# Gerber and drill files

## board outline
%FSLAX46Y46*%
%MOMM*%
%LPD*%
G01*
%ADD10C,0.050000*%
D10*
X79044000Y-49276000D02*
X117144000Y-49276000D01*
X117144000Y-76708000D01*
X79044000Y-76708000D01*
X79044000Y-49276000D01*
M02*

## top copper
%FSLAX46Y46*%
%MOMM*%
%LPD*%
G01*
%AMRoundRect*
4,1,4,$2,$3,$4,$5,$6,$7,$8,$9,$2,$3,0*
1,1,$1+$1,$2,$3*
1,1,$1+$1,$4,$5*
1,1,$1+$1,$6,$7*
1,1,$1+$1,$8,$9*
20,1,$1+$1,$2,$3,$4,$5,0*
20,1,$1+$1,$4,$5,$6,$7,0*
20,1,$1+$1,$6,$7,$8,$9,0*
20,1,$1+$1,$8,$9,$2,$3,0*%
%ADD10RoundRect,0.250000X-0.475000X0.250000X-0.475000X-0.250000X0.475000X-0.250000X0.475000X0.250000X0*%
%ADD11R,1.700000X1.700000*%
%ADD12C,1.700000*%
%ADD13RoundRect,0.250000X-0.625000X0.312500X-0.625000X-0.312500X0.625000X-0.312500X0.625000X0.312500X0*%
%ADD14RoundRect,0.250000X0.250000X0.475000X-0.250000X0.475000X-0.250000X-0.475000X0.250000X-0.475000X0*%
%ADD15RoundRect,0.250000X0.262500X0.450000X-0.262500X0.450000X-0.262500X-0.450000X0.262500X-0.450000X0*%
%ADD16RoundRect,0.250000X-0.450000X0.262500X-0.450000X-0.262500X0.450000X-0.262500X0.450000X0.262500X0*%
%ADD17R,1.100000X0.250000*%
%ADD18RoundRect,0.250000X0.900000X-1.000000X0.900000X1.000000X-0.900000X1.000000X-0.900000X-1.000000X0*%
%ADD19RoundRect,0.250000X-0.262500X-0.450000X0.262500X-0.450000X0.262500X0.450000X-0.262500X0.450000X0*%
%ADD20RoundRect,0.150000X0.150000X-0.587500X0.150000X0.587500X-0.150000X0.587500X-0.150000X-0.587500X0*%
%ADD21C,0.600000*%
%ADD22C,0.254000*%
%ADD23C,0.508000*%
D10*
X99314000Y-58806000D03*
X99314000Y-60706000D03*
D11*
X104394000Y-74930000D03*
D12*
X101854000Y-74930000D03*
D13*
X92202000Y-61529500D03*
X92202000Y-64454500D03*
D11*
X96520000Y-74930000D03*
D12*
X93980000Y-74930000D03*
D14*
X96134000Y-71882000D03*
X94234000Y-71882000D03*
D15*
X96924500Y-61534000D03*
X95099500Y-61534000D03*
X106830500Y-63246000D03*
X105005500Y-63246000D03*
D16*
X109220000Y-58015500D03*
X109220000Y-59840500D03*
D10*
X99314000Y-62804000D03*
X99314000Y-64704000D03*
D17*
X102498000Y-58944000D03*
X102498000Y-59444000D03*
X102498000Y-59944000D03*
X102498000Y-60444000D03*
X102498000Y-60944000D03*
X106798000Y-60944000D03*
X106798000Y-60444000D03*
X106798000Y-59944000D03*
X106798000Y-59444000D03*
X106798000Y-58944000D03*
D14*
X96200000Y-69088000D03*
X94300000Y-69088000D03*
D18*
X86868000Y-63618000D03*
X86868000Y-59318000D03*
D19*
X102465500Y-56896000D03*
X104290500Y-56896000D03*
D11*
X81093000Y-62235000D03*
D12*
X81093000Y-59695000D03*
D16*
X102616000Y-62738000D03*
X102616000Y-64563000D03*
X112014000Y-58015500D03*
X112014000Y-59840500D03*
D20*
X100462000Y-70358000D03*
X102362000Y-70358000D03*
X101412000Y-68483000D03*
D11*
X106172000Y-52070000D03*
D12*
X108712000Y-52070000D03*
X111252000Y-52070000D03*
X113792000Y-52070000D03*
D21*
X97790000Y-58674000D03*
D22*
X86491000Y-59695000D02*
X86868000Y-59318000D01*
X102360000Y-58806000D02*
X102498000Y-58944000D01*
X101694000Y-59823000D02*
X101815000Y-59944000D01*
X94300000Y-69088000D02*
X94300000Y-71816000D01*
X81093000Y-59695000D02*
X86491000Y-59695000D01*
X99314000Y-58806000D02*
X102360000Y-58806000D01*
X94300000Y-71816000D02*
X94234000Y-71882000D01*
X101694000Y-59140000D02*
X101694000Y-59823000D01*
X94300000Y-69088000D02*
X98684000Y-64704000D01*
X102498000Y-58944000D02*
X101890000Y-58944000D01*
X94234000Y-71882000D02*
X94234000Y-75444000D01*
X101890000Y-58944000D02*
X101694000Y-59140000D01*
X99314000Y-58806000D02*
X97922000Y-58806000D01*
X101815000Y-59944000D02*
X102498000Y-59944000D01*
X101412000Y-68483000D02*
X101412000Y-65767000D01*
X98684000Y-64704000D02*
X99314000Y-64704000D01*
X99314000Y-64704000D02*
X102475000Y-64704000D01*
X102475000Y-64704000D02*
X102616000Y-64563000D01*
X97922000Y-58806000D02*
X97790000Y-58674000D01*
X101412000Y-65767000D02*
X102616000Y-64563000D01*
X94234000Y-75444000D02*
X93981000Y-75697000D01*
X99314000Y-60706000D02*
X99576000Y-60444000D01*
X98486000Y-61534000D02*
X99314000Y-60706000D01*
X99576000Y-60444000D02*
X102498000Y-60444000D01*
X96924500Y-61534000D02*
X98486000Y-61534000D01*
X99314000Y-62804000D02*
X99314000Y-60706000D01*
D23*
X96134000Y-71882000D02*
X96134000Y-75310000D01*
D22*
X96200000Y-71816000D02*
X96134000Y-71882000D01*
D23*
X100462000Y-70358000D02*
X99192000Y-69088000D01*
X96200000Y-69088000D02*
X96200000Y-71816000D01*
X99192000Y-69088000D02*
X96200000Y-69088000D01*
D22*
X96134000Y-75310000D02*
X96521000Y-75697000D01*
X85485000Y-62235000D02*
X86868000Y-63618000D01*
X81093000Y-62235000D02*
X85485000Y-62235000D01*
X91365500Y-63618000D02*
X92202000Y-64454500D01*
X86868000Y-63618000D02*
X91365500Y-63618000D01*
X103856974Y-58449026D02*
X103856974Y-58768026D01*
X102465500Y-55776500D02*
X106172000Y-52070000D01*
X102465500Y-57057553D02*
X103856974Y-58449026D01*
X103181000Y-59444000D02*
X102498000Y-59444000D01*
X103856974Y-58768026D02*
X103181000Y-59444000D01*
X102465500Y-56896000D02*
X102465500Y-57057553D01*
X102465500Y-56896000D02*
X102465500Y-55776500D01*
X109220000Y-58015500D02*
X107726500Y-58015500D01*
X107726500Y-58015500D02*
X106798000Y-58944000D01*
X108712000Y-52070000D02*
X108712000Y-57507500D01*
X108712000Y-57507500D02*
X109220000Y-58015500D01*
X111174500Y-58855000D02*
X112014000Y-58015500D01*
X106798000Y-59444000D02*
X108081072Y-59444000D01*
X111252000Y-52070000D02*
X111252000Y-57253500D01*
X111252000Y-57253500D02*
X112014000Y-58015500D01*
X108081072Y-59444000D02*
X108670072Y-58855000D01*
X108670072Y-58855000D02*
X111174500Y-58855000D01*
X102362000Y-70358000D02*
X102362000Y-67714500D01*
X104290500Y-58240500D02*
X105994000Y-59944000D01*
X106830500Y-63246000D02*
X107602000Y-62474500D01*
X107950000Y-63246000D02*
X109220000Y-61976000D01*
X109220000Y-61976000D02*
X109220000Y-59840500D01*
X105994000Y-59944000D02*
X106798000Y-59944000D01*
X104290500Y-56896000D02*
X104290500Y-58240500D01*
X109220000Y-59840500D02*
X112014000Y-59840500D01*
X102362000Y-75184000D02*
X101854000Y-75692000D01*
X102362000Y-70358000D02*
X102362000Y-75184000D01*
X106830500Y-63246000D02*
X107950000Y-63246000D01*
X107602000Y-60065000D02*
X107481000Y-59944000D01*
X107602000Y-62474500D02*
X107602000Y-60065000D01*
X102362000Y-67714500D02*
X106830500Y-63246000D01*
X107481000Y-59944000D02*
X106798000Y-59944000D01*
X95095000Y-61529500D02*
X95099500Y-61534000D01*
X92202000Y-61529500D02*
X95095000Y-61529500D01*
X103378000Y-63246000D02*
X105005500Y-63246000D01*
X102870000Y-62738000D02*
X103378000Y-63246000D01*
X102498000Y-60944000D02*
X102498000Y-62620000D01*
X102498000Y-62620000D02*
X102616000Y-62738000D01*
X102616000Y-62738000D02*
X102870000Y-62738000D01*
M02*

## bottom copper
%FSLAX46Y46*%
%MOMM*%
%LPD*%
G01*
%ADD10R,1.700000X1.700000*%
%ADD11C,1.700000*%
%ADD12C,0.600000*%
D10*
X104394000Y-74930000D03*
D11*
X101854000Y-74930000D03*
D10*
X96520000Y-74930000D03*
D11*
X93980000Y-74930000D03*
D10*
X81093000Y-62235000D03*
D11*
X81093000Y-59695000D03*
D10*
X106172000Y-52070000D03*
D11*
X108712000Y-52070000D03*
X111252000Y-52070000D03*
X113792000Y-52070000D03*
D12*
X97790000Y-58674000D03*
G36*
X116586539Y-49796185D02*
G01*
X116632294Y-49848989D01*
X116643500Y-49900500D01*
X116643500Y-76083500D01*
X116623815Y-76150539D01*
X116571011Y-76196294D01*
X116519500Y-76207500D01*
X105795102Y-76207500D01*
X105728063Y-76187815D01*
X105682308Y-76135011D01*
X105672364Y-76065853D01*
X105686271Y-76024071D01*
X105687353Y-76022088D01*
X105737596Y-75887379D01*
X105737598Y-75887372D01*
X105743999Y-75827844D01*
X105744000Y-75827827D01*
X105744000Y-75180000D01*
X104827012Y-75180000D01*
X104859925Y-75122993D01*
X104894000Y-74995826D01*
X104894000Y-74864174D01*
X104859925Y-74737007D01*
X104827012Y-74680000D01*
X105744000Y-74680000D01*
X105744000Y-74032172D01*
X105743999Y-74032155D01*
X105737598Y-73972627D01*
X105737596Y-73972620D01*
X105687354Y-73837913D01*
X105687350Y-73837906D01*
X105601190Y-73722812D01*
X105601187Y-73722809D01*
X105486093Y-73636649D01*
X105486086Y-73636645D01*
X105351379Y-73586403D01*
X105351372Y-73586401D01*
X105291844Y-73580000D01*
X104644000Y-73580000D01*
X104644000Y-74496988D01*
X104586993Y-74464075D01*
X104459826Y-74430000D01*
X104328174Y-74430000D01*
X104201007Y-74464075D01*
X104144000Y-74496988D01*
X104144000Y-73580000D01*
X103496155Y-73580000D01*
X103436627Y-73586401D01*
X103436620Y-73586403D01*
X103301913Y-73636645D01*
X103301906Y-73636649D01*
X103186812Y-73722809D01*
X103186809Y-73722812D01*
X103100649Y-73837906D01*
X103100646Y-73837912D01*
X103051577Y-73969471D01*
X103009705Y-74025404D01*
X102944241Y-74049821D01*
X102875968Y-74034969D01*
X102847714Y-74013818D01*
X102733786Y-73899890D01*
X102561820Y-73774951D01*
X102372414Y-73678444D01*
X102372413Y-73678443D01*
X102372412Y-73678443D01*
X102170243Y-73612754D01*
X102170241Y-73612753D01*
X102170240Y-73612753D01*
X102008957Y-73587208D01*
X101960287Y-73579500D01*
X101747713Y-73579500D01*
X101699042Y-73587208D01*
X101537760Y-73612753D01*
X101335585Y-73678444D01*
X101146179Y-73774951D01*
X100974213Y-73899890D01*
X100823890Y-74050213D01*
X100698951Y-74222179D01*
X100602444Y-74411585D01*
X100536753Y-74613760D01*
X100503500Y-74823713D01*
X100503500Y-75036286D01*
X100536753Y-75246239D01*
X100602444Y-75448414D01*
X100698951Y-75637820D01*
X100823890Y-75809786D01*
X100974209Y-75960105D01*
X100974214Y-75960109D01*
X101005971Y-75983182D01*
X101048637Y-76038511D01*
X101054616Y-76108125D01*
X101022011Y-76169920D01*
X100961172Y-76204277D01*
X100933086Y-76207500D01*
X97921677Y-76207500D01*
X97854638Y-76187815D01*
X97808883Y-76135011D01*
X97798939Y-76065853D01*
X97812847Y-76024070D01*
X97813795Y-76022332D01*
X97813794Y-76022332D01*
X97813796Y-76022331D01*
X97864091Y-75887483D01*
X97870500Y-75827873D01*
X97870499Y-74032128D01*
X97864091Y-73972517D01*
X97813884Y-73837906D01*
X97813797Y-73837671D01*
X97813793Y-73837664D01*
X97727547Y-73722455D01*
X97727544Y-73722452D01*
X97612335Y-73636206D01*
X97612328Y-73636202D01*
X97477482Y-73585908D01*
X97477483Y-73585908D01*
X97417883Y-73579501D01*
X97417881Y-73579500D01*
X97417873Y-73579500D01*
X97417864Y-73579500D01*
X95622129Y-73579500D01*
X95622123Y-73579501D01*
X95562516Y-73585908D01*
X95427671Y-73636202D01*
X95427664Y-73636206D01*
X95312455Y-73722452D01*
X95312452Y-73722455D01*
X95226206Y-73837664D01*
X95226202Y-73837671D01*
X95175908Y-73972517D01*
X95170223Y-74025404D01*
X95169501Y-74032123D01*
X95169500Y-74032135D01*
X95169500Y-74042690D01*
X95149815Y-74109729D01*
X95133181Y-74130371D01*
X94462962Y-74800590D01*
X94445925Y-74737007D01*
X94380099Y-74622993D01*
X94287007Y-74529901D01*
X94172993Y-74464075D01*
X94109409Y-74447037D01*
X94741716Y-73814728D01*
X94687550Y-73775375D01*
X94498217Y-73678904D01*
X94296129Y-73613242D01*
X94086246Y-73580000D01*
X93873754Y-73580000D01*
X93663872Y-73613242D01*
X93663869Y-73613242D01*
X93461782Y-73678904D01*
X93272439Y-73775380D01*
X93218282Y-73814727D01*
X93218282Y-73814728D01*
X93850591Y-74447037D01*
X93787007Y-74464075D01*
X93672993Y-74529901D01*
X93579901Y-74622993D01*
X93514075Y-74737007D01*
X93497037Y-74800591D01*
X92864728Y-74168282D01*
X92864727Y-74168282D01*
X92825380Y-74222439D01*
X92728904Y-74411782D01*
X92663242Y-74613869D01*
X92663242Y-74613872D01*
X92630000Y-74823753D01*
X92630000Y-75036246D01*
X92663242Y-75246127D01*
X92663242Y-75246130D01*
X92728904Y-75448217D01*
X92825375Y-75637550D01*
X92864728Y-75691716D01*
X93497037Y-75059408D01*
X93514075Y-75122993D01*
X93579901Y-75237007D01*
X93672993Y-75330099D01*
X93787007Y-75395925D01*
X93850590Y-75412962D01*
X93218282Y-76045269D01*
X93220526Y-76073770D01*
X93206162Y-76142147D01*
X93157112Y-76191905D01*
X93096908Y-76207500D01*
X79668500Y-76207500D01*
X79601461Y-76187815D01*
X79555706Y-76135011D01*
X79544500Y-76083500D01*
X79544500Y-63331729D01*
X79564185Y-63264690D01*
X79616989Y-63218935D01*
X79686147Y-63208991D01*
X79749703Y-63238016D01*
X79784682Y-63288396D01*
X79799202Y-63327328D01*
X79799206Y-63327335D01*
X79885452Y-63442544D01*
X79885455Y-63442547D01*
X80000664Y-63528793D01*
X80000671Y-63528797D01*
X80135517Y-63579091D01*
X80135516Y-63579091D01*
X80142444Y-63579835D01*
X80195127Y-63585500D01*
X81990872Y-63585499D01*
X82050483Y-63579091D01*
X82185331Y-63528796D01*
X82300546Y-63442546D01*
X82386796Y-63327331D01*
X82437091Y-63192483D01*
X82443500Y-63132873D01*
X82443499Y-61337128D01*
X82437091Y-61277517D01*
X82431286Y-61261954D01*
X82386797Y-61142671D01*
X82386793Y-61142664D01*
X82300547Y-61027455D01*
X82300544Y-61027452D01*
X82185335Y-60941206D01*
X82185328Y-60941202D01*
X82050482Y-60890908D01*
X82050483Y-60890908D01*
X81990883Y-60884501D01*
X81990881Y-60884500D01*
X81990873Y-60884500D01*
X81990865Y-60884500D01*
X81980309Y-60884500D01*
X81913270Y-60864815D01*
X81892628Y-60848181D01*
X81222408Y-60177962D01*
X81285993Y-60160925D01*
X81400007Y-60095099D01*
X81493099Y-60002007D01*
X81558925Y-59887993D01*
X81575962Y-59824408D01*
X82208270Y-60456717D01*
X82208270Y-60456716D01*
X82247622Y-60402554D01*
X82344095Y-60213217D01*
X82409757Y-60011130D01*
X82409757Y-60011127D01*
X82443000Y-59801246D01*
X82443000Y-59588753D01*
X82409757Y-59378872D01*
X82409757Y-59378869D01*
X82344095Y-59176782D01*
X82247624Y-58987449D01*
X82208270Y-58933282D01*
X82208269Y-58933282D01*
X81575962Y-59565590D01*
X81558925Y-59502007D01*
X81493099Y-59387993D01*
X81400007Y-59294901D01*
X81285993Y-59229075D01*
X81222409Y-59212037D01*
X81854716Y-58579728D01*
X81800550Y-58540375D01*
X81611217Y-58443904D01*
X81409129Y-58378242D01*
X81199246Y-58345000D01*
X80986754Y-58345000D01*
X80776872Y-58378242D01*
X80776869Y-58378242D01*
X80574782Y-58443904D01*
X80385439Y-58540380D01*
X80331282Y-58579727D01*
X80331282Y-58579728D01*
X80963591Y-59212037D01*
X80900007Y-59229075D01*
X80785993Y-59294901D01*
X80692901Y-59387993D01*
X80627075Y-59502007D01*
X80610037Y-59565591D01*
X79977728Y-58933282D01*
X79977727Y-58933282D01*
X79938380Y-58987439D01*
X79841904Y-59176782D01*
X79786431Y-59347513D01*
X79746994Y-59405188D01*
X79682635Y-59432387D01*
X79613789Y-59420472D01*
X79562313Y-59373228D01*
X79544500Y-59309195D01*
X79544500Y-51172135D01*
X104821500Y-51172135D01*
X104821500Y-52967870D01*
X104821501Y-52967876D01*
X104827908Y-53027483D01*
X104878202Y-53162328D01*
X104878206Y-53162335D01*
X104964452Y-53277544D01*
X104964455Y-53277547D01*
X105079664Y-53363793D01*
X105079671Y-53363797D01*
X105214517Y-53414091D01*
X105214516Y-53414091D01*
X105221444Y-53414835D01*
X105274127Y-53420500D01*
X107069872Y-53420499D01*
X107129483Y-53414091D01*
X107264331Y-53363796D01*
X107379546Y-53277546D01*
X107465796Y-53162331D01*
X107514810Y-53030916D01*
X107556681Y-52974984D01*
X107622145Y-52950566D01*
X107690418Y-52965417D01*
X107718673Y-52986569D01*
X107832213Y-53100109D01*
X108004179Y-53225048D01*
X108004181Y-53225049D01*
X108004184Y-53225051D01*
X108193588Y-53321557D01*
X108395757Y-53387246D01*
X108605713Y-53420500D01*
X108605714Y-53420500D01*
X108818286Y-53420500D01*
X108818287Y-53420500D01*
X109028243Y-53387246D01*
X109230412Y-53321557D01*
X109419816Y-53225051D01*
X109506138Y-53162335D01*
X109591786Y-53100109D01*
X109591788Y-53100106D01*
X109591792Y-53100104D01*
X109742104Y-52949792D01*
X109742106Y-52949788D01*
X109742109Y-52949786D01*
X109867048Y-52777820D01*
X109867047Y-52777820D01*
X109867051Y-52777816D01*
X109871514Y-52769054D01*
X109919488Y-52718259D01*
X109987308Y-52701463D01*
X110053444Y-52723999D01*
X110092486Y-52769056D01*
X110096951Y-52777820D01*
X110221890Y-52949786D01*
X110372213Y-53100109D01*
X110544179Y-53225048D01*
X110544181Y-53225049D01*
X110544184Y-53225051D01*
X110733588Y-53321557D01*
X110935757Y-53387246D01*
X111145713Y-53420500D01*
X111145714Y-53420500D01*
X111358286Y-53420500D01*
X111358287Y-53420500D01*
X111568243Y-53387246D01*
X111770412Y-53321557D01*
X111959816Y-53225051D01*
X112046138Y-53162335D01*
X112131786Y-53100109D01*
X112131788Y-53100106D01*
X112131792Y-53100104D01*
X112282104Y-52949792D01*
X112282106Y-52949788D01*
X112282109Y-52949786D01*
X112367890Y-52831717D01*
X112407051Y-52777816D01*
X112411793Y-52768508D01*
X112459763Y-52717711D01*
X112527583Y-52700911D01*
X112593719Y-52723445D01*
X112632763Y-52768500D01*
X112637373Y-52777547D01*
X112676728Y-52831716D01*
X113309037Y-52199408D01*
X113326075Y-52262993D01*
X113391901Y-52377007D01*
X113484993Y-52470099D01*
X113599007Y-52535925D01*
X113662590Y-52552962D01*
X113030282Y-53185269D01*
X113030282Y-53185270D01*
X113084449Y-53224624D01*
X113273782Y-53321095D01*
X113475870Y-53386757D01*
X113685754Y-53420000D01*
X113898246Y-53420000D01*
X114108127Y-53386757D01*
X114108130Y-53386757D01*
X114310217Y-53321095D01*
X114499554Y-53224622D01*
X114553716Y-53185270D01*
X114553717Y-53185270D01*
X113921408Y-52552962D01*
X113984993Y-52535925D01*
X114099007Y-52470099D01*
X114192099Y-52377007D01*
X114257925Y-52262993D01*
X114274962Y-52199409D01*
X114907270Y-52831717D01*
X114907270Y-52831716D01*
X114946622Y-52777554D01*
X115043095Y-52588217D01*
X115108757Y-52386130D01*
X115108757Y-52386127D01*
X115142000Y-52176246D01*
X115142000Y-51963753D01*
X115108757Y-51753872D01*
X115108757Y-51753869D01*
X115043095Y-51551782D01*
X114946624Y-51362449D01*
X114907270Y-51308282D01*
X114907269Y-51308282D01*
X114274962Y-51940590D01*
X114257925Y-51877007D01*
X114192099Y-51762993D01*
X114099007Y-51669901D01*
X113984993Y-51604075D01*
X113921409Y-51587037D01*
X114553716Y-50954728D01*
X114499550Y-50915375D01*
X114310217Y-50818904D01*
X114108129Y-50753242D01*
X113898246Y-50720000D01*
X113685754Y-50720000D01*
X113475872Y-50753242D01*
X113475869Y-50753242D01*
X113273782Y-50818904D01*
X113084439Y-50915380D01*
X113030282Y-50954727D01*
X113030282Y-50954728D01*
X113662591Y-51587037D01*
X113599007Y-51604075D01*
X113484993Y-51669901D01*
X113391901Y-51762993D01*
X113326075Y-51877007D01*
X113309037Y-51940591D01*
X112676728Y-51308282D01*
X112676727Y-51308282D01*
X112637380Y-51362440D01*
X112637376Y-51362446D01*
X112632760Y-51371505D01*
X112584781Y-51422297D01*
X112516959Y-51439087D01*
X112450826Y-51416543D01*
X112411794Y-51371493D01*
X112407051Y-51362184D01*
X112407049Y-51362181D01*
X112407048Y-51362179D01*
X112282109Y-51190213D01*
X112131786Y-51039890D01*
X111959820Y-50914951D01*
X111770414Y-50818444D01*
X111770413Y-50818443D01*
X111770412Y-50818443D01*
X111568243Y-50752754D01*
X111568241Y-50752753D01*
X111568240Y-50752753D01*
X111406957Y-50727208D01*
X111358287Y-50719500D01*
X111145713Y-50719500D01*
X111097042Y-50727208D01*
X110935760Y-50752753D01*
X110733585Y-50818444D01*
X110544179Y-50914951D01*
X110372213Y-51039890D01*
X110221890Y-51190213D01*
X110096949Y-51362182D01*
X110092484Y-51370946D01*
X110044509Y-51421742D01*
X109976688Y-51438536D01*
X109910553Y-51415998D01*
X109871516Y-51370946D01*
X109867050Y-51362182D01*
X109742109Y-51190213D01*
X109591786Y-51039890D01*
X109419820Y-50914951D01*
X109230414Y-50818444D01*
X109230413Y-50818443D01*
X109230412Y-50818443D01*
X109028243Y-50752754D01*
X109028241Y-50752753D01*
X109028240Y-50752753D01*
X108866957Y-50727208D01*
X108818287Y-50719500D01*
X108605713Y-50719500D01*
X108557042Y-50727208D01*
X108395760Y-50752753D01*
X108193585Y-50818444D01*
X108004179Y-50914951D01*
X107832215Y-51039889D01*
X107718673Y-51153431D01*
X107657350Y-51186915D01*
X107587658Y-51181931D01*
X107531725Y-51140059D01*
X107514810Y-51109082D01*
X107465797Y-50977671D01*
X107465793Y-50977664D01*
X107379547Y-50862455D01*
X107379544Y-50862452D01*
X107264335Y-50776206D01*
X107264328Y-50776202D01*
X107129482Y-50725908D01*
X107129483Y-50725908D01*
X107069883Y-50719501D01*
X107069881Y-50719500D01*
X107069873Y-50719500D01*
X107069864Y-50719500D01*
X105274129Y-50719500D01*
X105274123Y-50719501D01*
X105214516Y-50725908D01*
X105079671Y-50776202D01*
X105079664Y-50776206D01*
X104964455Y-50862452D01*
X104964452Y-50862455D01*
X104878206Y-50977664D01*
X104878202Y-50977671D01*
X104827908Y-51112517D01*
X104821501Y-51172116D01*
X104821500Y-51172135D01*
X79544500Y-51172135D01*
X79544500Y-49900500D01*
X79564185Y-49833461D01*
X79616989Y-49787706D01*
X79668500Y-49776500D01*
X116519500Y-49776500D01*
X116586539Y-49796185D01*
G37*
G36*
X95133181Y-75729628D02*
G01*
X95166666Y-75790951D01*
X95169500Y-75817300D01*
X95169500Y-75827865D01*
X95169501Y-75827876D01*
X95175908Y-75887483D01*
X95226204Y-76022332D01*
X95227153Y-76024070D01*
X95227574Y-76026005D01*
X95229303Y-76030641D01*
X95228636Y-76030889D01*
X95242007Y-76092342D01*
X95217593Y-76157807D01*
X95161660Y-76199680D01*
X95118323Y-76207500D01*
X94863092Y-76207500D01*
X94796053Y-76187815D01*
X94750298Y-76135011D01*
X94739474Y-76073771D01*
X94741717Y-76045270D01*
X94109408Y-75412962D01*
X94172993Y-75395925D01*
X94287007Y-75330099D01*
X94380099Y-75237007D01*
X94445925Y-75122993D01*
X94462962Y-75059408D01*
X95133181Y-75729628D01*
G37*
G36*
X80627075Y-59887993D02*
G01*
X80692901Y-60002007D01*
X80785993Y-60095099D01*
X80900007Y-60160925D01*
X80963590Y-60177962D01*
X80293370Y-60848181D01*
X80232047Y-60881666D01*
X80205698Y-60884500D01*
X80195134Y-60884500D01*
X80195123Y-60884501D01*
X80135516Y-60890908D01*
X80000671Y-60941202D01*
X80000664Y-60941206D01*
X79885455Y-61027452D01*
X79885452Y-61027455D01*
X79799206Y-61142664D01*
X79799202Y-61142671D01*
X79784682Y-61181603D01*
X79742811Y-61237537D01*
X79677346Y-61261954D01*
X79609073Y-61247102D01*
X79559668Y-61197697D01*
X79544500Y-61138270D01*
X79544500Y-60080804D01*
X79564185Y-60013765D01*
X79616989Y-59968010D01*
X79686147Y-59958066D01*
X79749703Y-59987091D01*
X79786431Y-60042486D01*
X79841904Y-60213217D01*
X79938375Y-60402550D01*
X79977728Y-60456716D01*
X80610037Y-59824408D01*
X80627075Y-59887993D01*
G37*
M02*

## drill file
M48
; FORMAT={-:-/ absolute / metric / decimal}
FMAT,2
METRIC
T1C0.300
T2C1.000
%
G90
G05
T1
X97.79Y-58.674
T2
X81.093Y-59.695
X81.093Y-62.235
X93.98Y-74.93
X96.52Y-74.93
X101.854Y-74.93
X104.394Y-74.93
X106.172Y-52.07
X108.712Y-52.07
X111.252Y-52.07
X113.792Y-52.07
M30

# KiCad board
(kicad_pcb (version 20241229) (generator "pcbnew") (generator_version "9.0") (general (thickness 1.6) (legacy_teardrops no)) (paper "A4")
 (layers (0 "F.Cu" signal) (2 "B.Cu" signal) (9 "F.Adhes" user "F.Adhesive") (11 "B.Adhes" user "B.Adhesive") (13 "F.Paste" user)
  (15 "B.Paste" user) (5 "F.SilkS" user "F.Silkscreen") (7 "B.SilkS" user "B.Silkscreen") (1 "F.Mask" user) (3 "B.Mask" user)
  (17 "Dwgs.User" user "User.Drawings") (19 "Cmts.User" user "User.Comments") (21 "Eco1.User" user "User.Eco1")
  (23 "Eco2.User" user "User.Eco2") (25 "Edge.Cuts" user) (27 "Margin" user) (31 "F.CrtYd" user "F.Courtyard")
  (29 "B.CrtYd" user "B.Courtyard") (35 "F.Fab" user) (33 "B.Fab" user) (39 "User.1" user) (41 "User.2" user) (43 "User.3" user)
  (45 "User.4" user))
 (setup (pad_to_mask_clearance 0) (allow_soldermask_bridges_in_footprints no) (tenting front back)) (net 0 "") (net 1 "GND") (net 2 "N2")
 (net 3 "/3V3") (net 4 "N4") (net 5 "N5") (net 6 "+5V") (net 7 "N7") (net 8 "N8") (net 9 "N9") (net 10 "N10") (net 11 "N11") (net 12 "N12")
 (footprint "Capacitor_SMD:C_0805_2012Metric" (layer "F.Cu") (at 99.314 59.756 -90)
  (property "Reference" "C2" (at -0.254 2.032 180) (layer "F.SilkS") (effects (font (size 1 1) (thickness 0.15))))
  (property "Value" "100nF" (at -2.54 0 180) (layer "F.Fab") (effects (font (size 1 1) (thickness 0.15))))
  (pad "1" smd roundrect (at -0.95 0 270) (size 1 1.45) (layers "F.Cu" "F.Mask" "F.Paste") (roundrect_rratio 0.25) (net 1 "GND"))
  (pad "2" smd roundrect (at 0.95 0 270) (size 1 1.45) (layers "F.Cu" "F.Mask" "F.Paste") (roundrect_rratio 0.25) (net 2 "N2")))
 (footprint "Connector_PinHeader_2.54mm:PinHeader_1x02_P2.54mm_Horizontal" (layer "F.Cu") (at 104.394 74.93 -90)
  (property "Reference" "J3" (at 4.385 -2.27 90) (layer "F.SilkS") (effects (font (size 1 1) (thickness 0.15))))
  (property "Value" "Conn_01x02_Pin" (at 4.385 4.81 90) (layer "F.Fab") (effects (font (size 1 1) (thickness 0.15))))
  (pad "1" thru_hole rect (at 0 0 270) (size 1.7 1.7) (drill 1) (layers "*.Cu" "*.Mask") (remove_unused_layers no) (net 1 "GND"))
  (pad "2" thru_hole circle (at 0 2.54 270) (size 1.7 1.7) (drill 1) (layers "*.Cu" "*.Mask") (remove_unused_layers no) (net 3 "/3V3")))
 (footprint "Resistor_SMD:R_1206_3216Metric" (layer "F.Cu") (at 92.202 62.992 -90)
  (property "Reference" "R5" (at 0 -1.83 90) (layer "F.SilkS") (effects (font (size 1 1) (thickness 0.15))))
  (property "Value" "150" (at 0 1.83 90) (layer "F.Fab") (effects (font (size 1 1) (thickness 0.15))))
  (pad "1" smd roundrect (at -1.4625 0 270) (size 1.125 1.75) (layers "F.Cu" "F.Mask" "F.Paste") (roundrect_rratio 0.222222) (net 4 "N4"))
  (pad "2" smd roundrect (at 1.4625 0 270) (size 1.125 1.75) (layers "F.Cu" "F.Mask" "F.Paste") (roundrect_rratio 0.222222) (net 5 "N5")))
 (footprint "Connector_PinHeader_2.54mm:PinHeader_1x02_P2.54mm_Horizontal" (layer "F.Cu") (at 96.52 74.93 -90)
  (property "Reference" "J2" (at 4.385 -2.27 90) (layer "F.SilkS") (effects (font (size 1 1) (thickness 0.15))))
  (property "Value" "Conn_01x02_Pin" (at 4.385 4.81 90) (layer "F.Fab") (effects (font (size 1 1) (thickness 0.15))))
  (pad "1" thru_hole rect (at 0 0 270) (size 1.7 1.7) (drill 1) (layers "*.Cu" "*.Mask") (remove_unused_layers no) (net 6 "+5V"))
  (pad "2" thru_hole circle (at 0 2.54 270) (size 1.7 1.7) (drill 1) (layers "*.Cu" "*.Mask") (remove_unused_layers no) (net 1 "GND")))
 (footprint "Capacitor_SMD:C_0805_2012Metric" (layer "F.Cu") (at 95.184 71.882 180)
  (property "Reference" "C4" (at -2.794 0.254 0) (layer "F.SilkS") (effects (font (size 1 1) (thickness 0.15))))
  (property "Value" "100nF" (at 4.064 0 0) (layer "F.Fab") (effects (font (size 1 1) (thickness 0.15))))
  (pad "1" smd roundrect (at -0.95 0 180) (size 1 1.45) (layers "F.Cu" "F.Mask" "F.Paste") (roundrect_rratio 0.25) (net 6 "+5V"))
  (pad "2" smd roundrect (at 0.95 0 180) (size 1 1.45) (layers "F.Cu" "F.Mask" "F.Paste") (roundrect_rratio 0.25) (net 1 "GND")))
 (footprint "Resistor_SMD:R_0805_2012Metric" (layer "F.Cu") (at 96.012 61.534 180)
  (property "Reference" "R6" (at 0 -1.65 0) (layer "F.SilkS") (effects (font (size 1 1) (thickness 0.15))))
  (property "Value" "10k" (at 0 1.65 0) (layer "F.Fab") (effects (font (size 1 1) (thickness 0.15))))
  (pad "1" smd roundrect (at -0.9125 0 180) (size 1.025 1.4) (layers "F.Cu" "F.Mask" "F.Paste") (roundrect_rratio 0.243902) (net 2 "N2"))
  (pad "2" smd roundrect (at 0.9125 0 180) (size 1.025 1.4) (layers "F.Cu" "F.Mask" "F.Paste") (roundrect_rratio 0.243902) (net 4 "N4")))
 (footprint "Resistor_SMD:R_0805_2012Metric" (layer "F.Cu") (at 105.918 63.246 180)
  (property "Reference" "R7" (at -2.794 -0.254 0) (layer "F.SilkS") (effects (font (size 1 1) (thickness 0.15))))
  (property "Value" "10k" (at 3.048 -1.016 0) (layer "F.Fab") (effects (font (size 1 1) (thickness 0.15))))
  (pad "1" smd roundrect (at -0.9125 0 180) (size 1.025 1.4) (layers "F.Cu" "F.Mask" "F.Paste") (roundrect_rratio 0.243902) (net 3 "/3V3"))
  (pad "2" smd roundrect (at 0.9125 0 180) (size 1.025 1.4) (layers "F.Cu" "F.Mask" "F.Paste") (roundrect_rratio 0.243902) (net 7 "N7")))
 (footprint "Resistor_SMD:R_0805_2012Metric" (layer "F.Cu") (at 109.22 58.928 -90)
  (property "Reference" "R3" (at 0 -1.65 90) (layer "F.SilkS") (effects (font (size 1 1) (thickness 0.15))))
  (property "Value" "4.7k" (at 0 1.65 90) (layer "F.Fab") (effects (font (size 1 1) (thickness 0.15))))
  (pad "1" smd roundrect (at -0.9125 0 270) (size 1.025 1.4) (layers "F.Cu" "F.Mask" "F.Paste") (roundrect_rratio 0.243902) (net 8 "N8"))
  (pad "2" smd roundrect (at 0.9125 0 270) (size 1.025 1.4) (layers "F.Cu" "F.Mask" "F.Paste") (roundrect_rratio 0.243902) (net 3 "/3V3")))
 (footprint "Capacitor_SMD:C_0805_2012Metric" (layer "F.Cu") (at 99.314 63.754 -90)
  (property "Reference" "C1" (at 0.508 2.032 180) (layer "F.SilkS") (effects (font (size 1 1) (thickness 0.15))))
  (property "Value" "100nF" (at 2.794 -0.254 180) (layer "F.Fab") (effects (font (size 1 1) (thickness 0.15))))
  (pad "1" smd roundrect (at -0.95 0 270) (size 1 1.45) (layers "F.Cu" "F.Mask" "F.Paste") (roundrect_rratio 0.25) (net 2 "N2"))
  (pad "2" smd roundrect (at 0.95 0 270) (size 1 1.45) (layers "F.Cu" "F.Mask" "F.Paste") (roundrect_rratio 0.25) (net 1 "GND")))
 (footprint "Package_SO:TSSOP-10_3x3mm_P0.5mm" (layer "F.Cu") (at 104.648 59.944)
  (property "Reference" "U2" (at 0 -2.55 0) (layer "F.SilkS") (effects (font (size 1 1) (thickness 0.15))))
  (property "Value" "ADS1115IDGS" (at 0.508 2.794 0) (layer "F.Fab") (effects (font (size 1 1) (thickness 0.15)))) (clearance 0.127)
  (pad "1" smd rect (at -2.15 -1) (size 1.1 0.25) (layers "F.Cu" "F.Mask" "F.Paste") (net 1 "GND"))
  (pad "2" smd rect (at -2.15 -0.5) (size 1.1 0.25) (layers "F.Cu" "F.Mask" "F.Paste") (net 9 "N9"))
  (pad "3" smd rect (at -2.15 0) (size 1.1 0.25) (layers "F.Cu" "F.Mask" "F.Paste") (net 1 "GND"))
  (pad "4" smd rect (at -2.15 0.5) (size 1.1 0.25) (layers "F.Cu" "F.Mask" "F.Paste") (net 2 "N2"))
  (pad "5" smd rect (at -2.15 1) (size 1.1 0.25) (layers "F.Cu" "F.Mask" "F.Paste") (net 7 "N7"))
  (pad "6" smd rect (at 2.15 1) (size 1.1 0.25) (layers "F.Cu" "F.Mask" "F.Paste") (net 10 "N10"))
  (pad "7" smd rect (at 2.15 0.5) (size 1.1 0.25) (layers "F.Cu" "F.Mask" "F.Paste") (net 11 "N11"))
  (pad "8" smd rect (at 2.15 0) (size 1.1 0.25) (layers "F.Cu" "F.Mask" "F.Paste") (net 3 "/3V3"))
  (pad "9" smd rect (at 2.15 -0.5) (size 1.1 0.25) (layers "F.Cu" "F.Mask" "F.Paste") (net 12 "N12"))
  (pad "10" smd rect (at 2.15 -1) (size 1.1 0.25) (layers "F.Cu" "F.Mask" "F.Paste") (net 8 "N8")))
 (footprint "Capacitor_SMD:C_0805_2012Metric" (layer "F.Cu") (at 95.25 69.088 180)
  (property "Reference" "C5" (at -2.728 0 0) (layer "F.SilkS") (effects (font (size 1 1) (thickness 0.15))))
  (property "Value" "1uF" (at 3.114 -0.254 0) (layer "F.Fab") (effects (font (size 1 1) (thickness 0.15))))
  (pad "1" smd roundrect (at -0.95 0 180) (size 1 1.45) (layers "F.Cu" "F.Mask" "F.Paste") (roundrect_rratio 0.25) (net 6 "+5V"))
  (pad "2" smd roundrect (at 0.95 0 180) (size 1 1.45) (layers "F.Cu" "F.Mask" "F.Paste") (roundrect_rratio 0.25) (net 1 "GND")))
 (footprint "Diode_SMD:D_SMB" (layer "F.Cu") (at 86.868 61.468 90)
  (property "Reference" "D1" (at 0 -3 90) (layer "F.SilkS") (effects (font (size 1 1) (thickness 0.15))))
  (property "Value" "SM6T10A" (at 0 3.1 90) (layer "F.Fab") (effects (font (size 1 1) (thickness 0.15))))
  (pad "1" smd roundrect (at -2.15 0 90) (size 2.5 2.3) (layers "F.Cu" "F.Mask" "F.Paste") (roundrect_rratio 0.1086956522) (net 5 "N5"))
  (pad "2" smd roundrect (at 2.15 0 90) (size 2.5 2.3) (layers "F.Cu" "F.Mask" "F.Paste") (roundrect_rratio 0.1086956522) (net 1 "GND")))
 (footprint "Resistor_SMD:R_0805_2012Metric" (layer "F.Cu") (at 103.378 56.896)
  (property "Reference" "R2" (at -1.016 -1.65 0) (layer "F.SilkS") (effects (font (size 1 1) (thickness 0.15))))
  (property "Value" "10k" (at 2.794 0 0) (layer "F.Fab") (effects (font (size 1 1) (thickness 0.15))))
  (pad "1" smd roundrect (at -0.9125 0) (size 1.025 1.4) (layers "F.Cu" "F.Mask" "F.Paste") (roundrect_rratio 0.243902) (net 9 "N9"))
  (pad "2" smd roundrect (at 0.9125 0) (size 1.025 1.4) (layers "F.Cu" "F.Mask" "F.Paste") (roundrect_rratio 0.243902) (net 3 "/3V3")))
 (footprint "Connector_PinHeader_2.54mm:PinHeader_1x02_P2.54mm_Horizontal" (layer "F.Cu") (at 81.093 62.235 180)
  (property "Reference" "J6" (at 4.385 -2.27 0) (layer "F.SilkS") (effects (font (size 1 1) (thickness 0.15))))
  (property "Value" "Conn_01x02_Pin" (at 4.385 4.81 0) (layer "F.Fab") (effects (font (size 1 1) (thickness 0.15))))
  (pad "1" thru_hole rect (at 0 0 180) (size 1.7 1.7) (drill 1) (layers "*.Cu" "*.Mask") (remove_unused_layers no) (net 5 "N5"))
  (pad "2" thru_hole circle (at 0 2.54 180) (size 1.7 1.7) (drill 1) (layers "*.Cu" "*.Mask") (remove_unused_layers no) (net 1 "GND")))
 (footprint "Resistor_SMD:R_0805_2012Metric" (layer "F.Cu") (at 102.616 63.6505 -90)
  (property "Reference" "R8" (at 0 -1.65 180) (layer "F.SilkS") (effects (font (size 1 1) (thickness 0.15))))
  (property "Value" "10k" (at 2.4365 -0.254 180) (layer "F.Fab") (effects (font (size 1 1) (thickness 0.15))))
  (pad "1" smd roundrect (at -0.9125 0 270) (size 1.025 1.4) (layers "F.Cu" "F.Mask" "F.Paste") (roundrect_rratio 0.243902) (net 7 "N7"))
  (pad "2" smd roundrect (at 0.9125 0 270) (size 1.025 1.4) (layers "F.Cu" "F.Mask" "F.Paste") (roundrect_rratio 0.243902) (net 1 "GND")))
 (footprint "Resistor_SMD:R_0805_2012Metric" (layer "F.Cu") (at 112.014 58.928 -90)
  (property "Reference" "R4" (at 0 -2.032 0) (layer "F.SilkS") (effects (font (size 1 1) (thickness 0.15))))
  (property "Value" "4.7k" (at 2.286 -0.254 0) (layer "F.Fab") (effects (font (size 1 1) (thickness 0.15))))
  (pad "1" smd roundrect (at -0.9125 0 270) (size 1.025 1.4) (layers "F.Cu" "F.Mask" "F.Paste") (roundrect_rratio 0.243902) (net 12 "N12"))
  (pad "2" smd roundrect (at 0.9125 0 270) (size 1.025 1.4) (layers "F.Cu" "F.Mask" "F.Paste") (roundrect_rratio 0.243902) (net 3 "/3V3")))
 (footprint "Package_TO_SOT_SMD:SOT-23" (layer "F.Cu") (at 101.412 69.4205 90)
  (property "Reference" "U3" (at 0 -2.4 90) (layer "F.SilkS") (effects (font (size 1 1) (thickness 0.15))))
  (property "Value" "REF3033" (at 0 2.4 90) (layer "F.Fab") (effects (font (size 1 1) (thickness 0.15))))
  (pad "1" smd roundrect (at -0.9375 -0.95 90) (size 1.475 0.6) (layers "F.Cu" "F.Mask" "F.Paste") (roundrect_rratio 0.25) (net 6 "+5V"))
  (pad "2" smd roundrect (at -0.9375 0.95 90) (size 1.475 0.6) (layers "F.Cu" "F.Mask" "F.Paste") (roundrect_rratio 0.25) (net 3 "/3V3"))
  (pad "3" smd roundrect (at 0.9375 0 90) (size 1.475 0.6) (layers "F.Cu" "F.Mask" "F.Paste") (roundrect_rratio 0.25) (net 1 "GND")))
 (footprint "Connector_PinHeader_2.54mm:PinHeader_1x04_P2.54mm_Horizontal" (layer "F.Cu") (at 106.172 52.07 90)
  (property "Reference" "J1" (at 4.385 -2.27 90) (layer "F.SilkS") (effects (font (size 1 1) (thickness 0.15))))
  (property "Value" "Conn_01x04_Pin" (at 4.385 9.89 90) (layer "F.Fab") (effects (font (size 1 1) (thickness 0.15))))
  (pad "1" thru_hole rect (at 0 0 90) (size 1.7 1.7) (drill 1) (layers "*.Cu" "*.Mask") (remove_unused_layers no) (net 9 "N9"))
  (pad "2" thru_hole circle (at 0 2.54 90) (size 1.7 1.7) (drill 1) (layers "*.Cu" "*.Mask") (remove_unused_layers no) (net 8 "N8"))
  (pad "3" thru_hole circle (at 0 5.08 90) (size 1.7 1.7) (drill 1) (layers "*.Cu" "*.Mask") (remove_unused_layers no) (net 12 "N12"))
  (pad "4" thru_hole circle (at 0 7.62 90) (size 1.7 1.7) (drill 1) (layers "*.Cu" "*.Mask") (remove_unused_layers no) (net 1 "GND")))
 (gr_rect (start 79.044 49.276) (end 117.144 76.708) (stroke (width 0.05) (type default)) (fill no) (layer "Edge.Cuts"))
 (segment (start 86.491 59.695) (end 86.868 59.318) (width 0.254) (layer "F.Cu") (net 1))
 (segment (start 102.36 58.806) (end 102.498 58.944) (width 0.254) (layer "F.Cu") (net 1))
 (segment (start 101.694 59.823) (end 101.815 59.944) (width 0.254) (layer "F.Cu") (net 1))
 (segment (start 94.3 69.088) (end 94.3 71.816) (width 0.254) (layer "F.Cu") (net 1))
 (segment (start 81.093 59.695) (end 86.491 59.695) (width 0.254) (layer "F.Cu") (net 1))
 (segment (start 99.314 58.806) (end 102.36 58.806) (width 0.254) (layer "F.Cu") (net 1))
 (segment (start 94.3 71.816) (end 94.234 71.882) (width 0.254) (layer "F.Cu") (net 1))
 (segment (start 101.694 59.14) (end 101.694 59.823) (width 0.254) (layer "F.Cu") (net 1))
 (segment (start 94.3 69.088) (end 98.684 64.704) (width 0.254) (layer "F.Cu") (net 1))
 (segment (start 102.498 58.944) (end 101.89 58.944) (width 0.254) (layer "F.Cu") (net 1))
 (segment (start 94.234 71.882) (end 94.234 75.444) (width 0.254) (layer "F.Cu") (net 1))
 (segment (start 101.89 58.944) (end 101.694 59.14) (width 0.254) (layer "F.Cu") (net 1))
 (segment (start 99.314 58.806) (end 97.922 58.806) (width 0.254) (layer "F.Cu") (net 1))
 (segment (start 101.815 59.944) (end 102.498 59.944) (width 0.254) (layer "F.Cu") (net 1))
 (segment (start 101.412 68.483) (end 101.412 65.767) (width 0.254) (layer "F.Cu") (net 1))
 (segment (start 98.684 64.704) (end 99.314 64.704) (width 0.254) (layer "F.Cu") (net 1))
 (segment (start 99.314 64.704) (end 102.475 64.704) (width 0.254) (layer "F.Cu") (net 1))
 (segment (start 102.475 64.704) (end 102.616 64.563) (width 0.254) (layer "F.Cu") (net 1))
 (segment (start 97.922 58.806) (end 97.79 58.674) (width 0.254) (layer "F.Cu") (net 1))
 (segment (start 101.412 65.767) (end 102.616 64.563) (width 0.254) (layer "F.Cu") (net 1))
 (segment (start 94.234 75.444) (end 93.981 75.697) (width 0.254) (layer "F.Cu") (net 1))
 (via (at 97.79 58.674) (size 0.6) (drill 0.3) (layers "F.Cu" "B.Cu") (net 1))
 (segment (start 99.314 60.706) (end 99.576 60.444) (width 0.254) (layer "F.Cu") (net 2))
 (segment (start 98.486 61.534) (end 99.314 60.706) (width 0.254) (layer "F.Cu") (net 2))
 (segment (start 99.576 60.444) (end 102.498 60.444) (width 0.254) (layer "F.Cu") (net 2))
 (segment (start 96.9245 61.534) (end 98.486 61.534) (width 0.254) (layer "F.Cu") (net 2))
 (segment (start 99.314 62.804) (end 99.314 60.706) (width 0.254) (layer "F.Cu") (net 2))
 (segment (start 96.134 71.882) (end 96.134 75.31) (width 0.508) (layer "F.Cu") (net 6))
 (segment (start 96.2 71.816) (end 96.134 71.882) (width 0.254) (layer "F.Cu") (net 6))
 (segment (start 100.462 70.358) (end 99.192 69.088) (width 0.508) (layer "F.Cu") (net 6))
 (segment (start 96.2 69.088) (end 96.2 71.816) (width 0.508) (layer "F.Cu") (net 6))
 (segment (start 99.192 69.088) (end 96.2 69.088) (width 0.508) (layer "F.Cu") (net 6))
 (segment (start 96.134 75.31) (end 96.521 75.697) (width 0.254) (layer "F.Cu") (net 6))
 (segment (start 85.485 62.235) (end 86.868 63.618) (width 0.254) (layer "F.Cu") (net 5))
 (segment (start 81.093 62.235) (end 85.485 62.235) (width 0.254) (layer "F.Cu") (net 5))
 (segment (start 91.3655 63.618) (end 92.202 64.4545) (width 0.254) (layer "F.Cu") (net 5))
 (segment (start 86.868 63.618) (end 91.3655 63.618) (width 0.254) (layer "F.Cu") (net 5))
 (segment (start 103.856974 58.449026) (end 103.856974 58.768026) (width 0.254) (layer "F.Cu") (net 9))
 (segment (start 102.4655 55.7765) (end 106.172 52.07) (width 0.254) (layer "F.Cu") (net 9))
 (segment (start 102.4655 57.057553) (end 103.856974 58.449026) (width 0.254) (layer "F.Cu") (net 9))
 (segment (start 103.181 59.444) (end 102.498 59.444) (width 0.254) (layer "F.Cu") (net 9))
 (segment (start 103.856974 58.768026) (end 103.181 59.444) (width 0.254) (layer "F.Cu") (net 9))
 (segment (start 102.4655 56.896) (end 102.4655 57.057553) (width 0.254) (layer "F.Cu") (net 9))
 (segment (start 102.4655 56.896) (end 102.4655 55.7765) (width 0.254) (layer "F.Cu") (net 9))
 (segment (start 109.22 58.0155) (end 107.7265 58.0155) (width 0.254) (layer "F.Cu") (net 8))
 (segment (start 107.7265 58.0155) (end 106.798 58.944) (width 0.254) (layer "F.Cu") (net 8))
 (segment (start 108.712 52.07) (end 108.712 57.5075) (width 0.254) (layer "F.Cu") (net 8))
 (segment (start 108.712 57.5075) (end 109.22 58.0155) (width 0.254) (layer "F.Cu") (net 8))
 (segment (start 111.1745 58.855) (end 112.014 58.0155) (width 0.254) (layer "F.Cu") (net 12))
 (segment (start 106.798 59.444) (end 108.081072 59.444) (width 0.254) (layer "F.Cu") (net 12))
 (segment (start 111.252 52.07) (end 111.252 57.2535) (width 0.254) (layer "F.Cu") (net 12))
 (segment (start 111.252 57.2535) (end 112.014 58.0155) (width 0.254) (layer "F.Cu") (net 12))
 (segment (start 108.081072 59.444) (end 108.670072 58.855) (width 0.254) (layer "F.Cu") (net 12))
 (segment (start 108.670072 58.855) (end 111.1745 58.855) (width 0.254) (layer "F.Cu") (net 12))
 (segment (start 102.362 70.358) (end 102.362 67.7145) (width 0.254) (layer "F.Cu") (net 3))
 (segment (start 104.2905 58.2405) (end 105.994 59.944) (width 0.254) (layer "F.Cu") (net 3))
 (segment (start 106.8305 63.246) (end 107.602 62.4745) (width 0.254) (layer "F.Cu") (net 3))
 (segment (start 107.95 63.246) (end 109.22 61.976) (width 0.254) (layer "F.Cu") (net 3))
 (segment (start 109.22 61.976) (end 109.22 59.8405) (width 0.254) (layer "F.Cu") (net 3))
 (segment (start 105.994 59.944) (end 106.798 59.944) (width 0.254) (layer "F.Cu") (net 3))
 (segment (start 104.2905 56.896) (end 104.2905 58.2405) (width 0.254) (layer "F.Cu") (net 3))
 (segment (start 109.22 59.8405) (end 112.014 59.8405) (width 0.254) (layer "F.Cu") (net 3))
 (segment (start 102.362 75.184) (end 101.854 75.692) (width 0.254) (layer "F.Cu") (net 3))
 (segment (start 102.362 70.358) (end 102.362 75.184) (width 0.254) (layer "F.Cu") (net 3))
 (segment (start 106.8305 63.246) (end 107.95 63.246) (width 0.254) (layer "F.Cu") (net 3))
 (segment (start 107.602 60.065) (end 107.481 59.944) (width 0.254) (layer "F.Cu") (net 3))
 (segment (start 107.602 62.4745) (end 107.602 60.065) (width 0.254) (layer "F.Cu") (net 3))
 (segment (start 102.362 67.7145) (end 106.8305 63.246) (width 0.254) (layer "F.Cu") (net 3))
 (segment (start 107.481 59.944) (end 106.798 59.944) (width 0.254) (layer "F.Cu") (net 3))
 (segment (start 95.095 61.5295) (end 95.0995 61.534) (width 0.254) (layer "F.Cu") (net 4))
 (segment (start 92.202 61.5295) (end 95.095 61.5295) (width 0.254) (layer "F.Cu") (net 4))
 (segment (start 103.378 63.246) (end 105.0055 63.246) (width 0.254) (layer "F.Cu") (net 7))
 (segment (start 102.87 62.738) (end 103.378 63.246) (width 0.254) (layer "F.Cu") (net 7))
 (segment (start 102.498 60.944) (end 102.498 62.62) (width 0.254) (layer "F.Cu") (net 7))
 (segment (start 102.498 62.62) (end 102.616 62.738) (width 0.254) (layer "F.Cu") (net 7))
 (segment (start 102.616 62.738) (end 102.87 62.738) (width 0.254) (layer "F.Cu") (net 7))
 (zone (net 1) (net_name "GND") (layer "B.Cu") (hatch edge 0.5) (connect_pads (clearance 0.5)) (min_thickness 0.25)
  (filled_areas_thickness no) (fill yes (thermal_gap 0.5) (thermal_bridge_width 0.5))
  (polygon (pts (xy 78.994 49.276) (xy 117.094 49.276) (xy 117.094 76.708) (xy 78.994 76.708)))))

